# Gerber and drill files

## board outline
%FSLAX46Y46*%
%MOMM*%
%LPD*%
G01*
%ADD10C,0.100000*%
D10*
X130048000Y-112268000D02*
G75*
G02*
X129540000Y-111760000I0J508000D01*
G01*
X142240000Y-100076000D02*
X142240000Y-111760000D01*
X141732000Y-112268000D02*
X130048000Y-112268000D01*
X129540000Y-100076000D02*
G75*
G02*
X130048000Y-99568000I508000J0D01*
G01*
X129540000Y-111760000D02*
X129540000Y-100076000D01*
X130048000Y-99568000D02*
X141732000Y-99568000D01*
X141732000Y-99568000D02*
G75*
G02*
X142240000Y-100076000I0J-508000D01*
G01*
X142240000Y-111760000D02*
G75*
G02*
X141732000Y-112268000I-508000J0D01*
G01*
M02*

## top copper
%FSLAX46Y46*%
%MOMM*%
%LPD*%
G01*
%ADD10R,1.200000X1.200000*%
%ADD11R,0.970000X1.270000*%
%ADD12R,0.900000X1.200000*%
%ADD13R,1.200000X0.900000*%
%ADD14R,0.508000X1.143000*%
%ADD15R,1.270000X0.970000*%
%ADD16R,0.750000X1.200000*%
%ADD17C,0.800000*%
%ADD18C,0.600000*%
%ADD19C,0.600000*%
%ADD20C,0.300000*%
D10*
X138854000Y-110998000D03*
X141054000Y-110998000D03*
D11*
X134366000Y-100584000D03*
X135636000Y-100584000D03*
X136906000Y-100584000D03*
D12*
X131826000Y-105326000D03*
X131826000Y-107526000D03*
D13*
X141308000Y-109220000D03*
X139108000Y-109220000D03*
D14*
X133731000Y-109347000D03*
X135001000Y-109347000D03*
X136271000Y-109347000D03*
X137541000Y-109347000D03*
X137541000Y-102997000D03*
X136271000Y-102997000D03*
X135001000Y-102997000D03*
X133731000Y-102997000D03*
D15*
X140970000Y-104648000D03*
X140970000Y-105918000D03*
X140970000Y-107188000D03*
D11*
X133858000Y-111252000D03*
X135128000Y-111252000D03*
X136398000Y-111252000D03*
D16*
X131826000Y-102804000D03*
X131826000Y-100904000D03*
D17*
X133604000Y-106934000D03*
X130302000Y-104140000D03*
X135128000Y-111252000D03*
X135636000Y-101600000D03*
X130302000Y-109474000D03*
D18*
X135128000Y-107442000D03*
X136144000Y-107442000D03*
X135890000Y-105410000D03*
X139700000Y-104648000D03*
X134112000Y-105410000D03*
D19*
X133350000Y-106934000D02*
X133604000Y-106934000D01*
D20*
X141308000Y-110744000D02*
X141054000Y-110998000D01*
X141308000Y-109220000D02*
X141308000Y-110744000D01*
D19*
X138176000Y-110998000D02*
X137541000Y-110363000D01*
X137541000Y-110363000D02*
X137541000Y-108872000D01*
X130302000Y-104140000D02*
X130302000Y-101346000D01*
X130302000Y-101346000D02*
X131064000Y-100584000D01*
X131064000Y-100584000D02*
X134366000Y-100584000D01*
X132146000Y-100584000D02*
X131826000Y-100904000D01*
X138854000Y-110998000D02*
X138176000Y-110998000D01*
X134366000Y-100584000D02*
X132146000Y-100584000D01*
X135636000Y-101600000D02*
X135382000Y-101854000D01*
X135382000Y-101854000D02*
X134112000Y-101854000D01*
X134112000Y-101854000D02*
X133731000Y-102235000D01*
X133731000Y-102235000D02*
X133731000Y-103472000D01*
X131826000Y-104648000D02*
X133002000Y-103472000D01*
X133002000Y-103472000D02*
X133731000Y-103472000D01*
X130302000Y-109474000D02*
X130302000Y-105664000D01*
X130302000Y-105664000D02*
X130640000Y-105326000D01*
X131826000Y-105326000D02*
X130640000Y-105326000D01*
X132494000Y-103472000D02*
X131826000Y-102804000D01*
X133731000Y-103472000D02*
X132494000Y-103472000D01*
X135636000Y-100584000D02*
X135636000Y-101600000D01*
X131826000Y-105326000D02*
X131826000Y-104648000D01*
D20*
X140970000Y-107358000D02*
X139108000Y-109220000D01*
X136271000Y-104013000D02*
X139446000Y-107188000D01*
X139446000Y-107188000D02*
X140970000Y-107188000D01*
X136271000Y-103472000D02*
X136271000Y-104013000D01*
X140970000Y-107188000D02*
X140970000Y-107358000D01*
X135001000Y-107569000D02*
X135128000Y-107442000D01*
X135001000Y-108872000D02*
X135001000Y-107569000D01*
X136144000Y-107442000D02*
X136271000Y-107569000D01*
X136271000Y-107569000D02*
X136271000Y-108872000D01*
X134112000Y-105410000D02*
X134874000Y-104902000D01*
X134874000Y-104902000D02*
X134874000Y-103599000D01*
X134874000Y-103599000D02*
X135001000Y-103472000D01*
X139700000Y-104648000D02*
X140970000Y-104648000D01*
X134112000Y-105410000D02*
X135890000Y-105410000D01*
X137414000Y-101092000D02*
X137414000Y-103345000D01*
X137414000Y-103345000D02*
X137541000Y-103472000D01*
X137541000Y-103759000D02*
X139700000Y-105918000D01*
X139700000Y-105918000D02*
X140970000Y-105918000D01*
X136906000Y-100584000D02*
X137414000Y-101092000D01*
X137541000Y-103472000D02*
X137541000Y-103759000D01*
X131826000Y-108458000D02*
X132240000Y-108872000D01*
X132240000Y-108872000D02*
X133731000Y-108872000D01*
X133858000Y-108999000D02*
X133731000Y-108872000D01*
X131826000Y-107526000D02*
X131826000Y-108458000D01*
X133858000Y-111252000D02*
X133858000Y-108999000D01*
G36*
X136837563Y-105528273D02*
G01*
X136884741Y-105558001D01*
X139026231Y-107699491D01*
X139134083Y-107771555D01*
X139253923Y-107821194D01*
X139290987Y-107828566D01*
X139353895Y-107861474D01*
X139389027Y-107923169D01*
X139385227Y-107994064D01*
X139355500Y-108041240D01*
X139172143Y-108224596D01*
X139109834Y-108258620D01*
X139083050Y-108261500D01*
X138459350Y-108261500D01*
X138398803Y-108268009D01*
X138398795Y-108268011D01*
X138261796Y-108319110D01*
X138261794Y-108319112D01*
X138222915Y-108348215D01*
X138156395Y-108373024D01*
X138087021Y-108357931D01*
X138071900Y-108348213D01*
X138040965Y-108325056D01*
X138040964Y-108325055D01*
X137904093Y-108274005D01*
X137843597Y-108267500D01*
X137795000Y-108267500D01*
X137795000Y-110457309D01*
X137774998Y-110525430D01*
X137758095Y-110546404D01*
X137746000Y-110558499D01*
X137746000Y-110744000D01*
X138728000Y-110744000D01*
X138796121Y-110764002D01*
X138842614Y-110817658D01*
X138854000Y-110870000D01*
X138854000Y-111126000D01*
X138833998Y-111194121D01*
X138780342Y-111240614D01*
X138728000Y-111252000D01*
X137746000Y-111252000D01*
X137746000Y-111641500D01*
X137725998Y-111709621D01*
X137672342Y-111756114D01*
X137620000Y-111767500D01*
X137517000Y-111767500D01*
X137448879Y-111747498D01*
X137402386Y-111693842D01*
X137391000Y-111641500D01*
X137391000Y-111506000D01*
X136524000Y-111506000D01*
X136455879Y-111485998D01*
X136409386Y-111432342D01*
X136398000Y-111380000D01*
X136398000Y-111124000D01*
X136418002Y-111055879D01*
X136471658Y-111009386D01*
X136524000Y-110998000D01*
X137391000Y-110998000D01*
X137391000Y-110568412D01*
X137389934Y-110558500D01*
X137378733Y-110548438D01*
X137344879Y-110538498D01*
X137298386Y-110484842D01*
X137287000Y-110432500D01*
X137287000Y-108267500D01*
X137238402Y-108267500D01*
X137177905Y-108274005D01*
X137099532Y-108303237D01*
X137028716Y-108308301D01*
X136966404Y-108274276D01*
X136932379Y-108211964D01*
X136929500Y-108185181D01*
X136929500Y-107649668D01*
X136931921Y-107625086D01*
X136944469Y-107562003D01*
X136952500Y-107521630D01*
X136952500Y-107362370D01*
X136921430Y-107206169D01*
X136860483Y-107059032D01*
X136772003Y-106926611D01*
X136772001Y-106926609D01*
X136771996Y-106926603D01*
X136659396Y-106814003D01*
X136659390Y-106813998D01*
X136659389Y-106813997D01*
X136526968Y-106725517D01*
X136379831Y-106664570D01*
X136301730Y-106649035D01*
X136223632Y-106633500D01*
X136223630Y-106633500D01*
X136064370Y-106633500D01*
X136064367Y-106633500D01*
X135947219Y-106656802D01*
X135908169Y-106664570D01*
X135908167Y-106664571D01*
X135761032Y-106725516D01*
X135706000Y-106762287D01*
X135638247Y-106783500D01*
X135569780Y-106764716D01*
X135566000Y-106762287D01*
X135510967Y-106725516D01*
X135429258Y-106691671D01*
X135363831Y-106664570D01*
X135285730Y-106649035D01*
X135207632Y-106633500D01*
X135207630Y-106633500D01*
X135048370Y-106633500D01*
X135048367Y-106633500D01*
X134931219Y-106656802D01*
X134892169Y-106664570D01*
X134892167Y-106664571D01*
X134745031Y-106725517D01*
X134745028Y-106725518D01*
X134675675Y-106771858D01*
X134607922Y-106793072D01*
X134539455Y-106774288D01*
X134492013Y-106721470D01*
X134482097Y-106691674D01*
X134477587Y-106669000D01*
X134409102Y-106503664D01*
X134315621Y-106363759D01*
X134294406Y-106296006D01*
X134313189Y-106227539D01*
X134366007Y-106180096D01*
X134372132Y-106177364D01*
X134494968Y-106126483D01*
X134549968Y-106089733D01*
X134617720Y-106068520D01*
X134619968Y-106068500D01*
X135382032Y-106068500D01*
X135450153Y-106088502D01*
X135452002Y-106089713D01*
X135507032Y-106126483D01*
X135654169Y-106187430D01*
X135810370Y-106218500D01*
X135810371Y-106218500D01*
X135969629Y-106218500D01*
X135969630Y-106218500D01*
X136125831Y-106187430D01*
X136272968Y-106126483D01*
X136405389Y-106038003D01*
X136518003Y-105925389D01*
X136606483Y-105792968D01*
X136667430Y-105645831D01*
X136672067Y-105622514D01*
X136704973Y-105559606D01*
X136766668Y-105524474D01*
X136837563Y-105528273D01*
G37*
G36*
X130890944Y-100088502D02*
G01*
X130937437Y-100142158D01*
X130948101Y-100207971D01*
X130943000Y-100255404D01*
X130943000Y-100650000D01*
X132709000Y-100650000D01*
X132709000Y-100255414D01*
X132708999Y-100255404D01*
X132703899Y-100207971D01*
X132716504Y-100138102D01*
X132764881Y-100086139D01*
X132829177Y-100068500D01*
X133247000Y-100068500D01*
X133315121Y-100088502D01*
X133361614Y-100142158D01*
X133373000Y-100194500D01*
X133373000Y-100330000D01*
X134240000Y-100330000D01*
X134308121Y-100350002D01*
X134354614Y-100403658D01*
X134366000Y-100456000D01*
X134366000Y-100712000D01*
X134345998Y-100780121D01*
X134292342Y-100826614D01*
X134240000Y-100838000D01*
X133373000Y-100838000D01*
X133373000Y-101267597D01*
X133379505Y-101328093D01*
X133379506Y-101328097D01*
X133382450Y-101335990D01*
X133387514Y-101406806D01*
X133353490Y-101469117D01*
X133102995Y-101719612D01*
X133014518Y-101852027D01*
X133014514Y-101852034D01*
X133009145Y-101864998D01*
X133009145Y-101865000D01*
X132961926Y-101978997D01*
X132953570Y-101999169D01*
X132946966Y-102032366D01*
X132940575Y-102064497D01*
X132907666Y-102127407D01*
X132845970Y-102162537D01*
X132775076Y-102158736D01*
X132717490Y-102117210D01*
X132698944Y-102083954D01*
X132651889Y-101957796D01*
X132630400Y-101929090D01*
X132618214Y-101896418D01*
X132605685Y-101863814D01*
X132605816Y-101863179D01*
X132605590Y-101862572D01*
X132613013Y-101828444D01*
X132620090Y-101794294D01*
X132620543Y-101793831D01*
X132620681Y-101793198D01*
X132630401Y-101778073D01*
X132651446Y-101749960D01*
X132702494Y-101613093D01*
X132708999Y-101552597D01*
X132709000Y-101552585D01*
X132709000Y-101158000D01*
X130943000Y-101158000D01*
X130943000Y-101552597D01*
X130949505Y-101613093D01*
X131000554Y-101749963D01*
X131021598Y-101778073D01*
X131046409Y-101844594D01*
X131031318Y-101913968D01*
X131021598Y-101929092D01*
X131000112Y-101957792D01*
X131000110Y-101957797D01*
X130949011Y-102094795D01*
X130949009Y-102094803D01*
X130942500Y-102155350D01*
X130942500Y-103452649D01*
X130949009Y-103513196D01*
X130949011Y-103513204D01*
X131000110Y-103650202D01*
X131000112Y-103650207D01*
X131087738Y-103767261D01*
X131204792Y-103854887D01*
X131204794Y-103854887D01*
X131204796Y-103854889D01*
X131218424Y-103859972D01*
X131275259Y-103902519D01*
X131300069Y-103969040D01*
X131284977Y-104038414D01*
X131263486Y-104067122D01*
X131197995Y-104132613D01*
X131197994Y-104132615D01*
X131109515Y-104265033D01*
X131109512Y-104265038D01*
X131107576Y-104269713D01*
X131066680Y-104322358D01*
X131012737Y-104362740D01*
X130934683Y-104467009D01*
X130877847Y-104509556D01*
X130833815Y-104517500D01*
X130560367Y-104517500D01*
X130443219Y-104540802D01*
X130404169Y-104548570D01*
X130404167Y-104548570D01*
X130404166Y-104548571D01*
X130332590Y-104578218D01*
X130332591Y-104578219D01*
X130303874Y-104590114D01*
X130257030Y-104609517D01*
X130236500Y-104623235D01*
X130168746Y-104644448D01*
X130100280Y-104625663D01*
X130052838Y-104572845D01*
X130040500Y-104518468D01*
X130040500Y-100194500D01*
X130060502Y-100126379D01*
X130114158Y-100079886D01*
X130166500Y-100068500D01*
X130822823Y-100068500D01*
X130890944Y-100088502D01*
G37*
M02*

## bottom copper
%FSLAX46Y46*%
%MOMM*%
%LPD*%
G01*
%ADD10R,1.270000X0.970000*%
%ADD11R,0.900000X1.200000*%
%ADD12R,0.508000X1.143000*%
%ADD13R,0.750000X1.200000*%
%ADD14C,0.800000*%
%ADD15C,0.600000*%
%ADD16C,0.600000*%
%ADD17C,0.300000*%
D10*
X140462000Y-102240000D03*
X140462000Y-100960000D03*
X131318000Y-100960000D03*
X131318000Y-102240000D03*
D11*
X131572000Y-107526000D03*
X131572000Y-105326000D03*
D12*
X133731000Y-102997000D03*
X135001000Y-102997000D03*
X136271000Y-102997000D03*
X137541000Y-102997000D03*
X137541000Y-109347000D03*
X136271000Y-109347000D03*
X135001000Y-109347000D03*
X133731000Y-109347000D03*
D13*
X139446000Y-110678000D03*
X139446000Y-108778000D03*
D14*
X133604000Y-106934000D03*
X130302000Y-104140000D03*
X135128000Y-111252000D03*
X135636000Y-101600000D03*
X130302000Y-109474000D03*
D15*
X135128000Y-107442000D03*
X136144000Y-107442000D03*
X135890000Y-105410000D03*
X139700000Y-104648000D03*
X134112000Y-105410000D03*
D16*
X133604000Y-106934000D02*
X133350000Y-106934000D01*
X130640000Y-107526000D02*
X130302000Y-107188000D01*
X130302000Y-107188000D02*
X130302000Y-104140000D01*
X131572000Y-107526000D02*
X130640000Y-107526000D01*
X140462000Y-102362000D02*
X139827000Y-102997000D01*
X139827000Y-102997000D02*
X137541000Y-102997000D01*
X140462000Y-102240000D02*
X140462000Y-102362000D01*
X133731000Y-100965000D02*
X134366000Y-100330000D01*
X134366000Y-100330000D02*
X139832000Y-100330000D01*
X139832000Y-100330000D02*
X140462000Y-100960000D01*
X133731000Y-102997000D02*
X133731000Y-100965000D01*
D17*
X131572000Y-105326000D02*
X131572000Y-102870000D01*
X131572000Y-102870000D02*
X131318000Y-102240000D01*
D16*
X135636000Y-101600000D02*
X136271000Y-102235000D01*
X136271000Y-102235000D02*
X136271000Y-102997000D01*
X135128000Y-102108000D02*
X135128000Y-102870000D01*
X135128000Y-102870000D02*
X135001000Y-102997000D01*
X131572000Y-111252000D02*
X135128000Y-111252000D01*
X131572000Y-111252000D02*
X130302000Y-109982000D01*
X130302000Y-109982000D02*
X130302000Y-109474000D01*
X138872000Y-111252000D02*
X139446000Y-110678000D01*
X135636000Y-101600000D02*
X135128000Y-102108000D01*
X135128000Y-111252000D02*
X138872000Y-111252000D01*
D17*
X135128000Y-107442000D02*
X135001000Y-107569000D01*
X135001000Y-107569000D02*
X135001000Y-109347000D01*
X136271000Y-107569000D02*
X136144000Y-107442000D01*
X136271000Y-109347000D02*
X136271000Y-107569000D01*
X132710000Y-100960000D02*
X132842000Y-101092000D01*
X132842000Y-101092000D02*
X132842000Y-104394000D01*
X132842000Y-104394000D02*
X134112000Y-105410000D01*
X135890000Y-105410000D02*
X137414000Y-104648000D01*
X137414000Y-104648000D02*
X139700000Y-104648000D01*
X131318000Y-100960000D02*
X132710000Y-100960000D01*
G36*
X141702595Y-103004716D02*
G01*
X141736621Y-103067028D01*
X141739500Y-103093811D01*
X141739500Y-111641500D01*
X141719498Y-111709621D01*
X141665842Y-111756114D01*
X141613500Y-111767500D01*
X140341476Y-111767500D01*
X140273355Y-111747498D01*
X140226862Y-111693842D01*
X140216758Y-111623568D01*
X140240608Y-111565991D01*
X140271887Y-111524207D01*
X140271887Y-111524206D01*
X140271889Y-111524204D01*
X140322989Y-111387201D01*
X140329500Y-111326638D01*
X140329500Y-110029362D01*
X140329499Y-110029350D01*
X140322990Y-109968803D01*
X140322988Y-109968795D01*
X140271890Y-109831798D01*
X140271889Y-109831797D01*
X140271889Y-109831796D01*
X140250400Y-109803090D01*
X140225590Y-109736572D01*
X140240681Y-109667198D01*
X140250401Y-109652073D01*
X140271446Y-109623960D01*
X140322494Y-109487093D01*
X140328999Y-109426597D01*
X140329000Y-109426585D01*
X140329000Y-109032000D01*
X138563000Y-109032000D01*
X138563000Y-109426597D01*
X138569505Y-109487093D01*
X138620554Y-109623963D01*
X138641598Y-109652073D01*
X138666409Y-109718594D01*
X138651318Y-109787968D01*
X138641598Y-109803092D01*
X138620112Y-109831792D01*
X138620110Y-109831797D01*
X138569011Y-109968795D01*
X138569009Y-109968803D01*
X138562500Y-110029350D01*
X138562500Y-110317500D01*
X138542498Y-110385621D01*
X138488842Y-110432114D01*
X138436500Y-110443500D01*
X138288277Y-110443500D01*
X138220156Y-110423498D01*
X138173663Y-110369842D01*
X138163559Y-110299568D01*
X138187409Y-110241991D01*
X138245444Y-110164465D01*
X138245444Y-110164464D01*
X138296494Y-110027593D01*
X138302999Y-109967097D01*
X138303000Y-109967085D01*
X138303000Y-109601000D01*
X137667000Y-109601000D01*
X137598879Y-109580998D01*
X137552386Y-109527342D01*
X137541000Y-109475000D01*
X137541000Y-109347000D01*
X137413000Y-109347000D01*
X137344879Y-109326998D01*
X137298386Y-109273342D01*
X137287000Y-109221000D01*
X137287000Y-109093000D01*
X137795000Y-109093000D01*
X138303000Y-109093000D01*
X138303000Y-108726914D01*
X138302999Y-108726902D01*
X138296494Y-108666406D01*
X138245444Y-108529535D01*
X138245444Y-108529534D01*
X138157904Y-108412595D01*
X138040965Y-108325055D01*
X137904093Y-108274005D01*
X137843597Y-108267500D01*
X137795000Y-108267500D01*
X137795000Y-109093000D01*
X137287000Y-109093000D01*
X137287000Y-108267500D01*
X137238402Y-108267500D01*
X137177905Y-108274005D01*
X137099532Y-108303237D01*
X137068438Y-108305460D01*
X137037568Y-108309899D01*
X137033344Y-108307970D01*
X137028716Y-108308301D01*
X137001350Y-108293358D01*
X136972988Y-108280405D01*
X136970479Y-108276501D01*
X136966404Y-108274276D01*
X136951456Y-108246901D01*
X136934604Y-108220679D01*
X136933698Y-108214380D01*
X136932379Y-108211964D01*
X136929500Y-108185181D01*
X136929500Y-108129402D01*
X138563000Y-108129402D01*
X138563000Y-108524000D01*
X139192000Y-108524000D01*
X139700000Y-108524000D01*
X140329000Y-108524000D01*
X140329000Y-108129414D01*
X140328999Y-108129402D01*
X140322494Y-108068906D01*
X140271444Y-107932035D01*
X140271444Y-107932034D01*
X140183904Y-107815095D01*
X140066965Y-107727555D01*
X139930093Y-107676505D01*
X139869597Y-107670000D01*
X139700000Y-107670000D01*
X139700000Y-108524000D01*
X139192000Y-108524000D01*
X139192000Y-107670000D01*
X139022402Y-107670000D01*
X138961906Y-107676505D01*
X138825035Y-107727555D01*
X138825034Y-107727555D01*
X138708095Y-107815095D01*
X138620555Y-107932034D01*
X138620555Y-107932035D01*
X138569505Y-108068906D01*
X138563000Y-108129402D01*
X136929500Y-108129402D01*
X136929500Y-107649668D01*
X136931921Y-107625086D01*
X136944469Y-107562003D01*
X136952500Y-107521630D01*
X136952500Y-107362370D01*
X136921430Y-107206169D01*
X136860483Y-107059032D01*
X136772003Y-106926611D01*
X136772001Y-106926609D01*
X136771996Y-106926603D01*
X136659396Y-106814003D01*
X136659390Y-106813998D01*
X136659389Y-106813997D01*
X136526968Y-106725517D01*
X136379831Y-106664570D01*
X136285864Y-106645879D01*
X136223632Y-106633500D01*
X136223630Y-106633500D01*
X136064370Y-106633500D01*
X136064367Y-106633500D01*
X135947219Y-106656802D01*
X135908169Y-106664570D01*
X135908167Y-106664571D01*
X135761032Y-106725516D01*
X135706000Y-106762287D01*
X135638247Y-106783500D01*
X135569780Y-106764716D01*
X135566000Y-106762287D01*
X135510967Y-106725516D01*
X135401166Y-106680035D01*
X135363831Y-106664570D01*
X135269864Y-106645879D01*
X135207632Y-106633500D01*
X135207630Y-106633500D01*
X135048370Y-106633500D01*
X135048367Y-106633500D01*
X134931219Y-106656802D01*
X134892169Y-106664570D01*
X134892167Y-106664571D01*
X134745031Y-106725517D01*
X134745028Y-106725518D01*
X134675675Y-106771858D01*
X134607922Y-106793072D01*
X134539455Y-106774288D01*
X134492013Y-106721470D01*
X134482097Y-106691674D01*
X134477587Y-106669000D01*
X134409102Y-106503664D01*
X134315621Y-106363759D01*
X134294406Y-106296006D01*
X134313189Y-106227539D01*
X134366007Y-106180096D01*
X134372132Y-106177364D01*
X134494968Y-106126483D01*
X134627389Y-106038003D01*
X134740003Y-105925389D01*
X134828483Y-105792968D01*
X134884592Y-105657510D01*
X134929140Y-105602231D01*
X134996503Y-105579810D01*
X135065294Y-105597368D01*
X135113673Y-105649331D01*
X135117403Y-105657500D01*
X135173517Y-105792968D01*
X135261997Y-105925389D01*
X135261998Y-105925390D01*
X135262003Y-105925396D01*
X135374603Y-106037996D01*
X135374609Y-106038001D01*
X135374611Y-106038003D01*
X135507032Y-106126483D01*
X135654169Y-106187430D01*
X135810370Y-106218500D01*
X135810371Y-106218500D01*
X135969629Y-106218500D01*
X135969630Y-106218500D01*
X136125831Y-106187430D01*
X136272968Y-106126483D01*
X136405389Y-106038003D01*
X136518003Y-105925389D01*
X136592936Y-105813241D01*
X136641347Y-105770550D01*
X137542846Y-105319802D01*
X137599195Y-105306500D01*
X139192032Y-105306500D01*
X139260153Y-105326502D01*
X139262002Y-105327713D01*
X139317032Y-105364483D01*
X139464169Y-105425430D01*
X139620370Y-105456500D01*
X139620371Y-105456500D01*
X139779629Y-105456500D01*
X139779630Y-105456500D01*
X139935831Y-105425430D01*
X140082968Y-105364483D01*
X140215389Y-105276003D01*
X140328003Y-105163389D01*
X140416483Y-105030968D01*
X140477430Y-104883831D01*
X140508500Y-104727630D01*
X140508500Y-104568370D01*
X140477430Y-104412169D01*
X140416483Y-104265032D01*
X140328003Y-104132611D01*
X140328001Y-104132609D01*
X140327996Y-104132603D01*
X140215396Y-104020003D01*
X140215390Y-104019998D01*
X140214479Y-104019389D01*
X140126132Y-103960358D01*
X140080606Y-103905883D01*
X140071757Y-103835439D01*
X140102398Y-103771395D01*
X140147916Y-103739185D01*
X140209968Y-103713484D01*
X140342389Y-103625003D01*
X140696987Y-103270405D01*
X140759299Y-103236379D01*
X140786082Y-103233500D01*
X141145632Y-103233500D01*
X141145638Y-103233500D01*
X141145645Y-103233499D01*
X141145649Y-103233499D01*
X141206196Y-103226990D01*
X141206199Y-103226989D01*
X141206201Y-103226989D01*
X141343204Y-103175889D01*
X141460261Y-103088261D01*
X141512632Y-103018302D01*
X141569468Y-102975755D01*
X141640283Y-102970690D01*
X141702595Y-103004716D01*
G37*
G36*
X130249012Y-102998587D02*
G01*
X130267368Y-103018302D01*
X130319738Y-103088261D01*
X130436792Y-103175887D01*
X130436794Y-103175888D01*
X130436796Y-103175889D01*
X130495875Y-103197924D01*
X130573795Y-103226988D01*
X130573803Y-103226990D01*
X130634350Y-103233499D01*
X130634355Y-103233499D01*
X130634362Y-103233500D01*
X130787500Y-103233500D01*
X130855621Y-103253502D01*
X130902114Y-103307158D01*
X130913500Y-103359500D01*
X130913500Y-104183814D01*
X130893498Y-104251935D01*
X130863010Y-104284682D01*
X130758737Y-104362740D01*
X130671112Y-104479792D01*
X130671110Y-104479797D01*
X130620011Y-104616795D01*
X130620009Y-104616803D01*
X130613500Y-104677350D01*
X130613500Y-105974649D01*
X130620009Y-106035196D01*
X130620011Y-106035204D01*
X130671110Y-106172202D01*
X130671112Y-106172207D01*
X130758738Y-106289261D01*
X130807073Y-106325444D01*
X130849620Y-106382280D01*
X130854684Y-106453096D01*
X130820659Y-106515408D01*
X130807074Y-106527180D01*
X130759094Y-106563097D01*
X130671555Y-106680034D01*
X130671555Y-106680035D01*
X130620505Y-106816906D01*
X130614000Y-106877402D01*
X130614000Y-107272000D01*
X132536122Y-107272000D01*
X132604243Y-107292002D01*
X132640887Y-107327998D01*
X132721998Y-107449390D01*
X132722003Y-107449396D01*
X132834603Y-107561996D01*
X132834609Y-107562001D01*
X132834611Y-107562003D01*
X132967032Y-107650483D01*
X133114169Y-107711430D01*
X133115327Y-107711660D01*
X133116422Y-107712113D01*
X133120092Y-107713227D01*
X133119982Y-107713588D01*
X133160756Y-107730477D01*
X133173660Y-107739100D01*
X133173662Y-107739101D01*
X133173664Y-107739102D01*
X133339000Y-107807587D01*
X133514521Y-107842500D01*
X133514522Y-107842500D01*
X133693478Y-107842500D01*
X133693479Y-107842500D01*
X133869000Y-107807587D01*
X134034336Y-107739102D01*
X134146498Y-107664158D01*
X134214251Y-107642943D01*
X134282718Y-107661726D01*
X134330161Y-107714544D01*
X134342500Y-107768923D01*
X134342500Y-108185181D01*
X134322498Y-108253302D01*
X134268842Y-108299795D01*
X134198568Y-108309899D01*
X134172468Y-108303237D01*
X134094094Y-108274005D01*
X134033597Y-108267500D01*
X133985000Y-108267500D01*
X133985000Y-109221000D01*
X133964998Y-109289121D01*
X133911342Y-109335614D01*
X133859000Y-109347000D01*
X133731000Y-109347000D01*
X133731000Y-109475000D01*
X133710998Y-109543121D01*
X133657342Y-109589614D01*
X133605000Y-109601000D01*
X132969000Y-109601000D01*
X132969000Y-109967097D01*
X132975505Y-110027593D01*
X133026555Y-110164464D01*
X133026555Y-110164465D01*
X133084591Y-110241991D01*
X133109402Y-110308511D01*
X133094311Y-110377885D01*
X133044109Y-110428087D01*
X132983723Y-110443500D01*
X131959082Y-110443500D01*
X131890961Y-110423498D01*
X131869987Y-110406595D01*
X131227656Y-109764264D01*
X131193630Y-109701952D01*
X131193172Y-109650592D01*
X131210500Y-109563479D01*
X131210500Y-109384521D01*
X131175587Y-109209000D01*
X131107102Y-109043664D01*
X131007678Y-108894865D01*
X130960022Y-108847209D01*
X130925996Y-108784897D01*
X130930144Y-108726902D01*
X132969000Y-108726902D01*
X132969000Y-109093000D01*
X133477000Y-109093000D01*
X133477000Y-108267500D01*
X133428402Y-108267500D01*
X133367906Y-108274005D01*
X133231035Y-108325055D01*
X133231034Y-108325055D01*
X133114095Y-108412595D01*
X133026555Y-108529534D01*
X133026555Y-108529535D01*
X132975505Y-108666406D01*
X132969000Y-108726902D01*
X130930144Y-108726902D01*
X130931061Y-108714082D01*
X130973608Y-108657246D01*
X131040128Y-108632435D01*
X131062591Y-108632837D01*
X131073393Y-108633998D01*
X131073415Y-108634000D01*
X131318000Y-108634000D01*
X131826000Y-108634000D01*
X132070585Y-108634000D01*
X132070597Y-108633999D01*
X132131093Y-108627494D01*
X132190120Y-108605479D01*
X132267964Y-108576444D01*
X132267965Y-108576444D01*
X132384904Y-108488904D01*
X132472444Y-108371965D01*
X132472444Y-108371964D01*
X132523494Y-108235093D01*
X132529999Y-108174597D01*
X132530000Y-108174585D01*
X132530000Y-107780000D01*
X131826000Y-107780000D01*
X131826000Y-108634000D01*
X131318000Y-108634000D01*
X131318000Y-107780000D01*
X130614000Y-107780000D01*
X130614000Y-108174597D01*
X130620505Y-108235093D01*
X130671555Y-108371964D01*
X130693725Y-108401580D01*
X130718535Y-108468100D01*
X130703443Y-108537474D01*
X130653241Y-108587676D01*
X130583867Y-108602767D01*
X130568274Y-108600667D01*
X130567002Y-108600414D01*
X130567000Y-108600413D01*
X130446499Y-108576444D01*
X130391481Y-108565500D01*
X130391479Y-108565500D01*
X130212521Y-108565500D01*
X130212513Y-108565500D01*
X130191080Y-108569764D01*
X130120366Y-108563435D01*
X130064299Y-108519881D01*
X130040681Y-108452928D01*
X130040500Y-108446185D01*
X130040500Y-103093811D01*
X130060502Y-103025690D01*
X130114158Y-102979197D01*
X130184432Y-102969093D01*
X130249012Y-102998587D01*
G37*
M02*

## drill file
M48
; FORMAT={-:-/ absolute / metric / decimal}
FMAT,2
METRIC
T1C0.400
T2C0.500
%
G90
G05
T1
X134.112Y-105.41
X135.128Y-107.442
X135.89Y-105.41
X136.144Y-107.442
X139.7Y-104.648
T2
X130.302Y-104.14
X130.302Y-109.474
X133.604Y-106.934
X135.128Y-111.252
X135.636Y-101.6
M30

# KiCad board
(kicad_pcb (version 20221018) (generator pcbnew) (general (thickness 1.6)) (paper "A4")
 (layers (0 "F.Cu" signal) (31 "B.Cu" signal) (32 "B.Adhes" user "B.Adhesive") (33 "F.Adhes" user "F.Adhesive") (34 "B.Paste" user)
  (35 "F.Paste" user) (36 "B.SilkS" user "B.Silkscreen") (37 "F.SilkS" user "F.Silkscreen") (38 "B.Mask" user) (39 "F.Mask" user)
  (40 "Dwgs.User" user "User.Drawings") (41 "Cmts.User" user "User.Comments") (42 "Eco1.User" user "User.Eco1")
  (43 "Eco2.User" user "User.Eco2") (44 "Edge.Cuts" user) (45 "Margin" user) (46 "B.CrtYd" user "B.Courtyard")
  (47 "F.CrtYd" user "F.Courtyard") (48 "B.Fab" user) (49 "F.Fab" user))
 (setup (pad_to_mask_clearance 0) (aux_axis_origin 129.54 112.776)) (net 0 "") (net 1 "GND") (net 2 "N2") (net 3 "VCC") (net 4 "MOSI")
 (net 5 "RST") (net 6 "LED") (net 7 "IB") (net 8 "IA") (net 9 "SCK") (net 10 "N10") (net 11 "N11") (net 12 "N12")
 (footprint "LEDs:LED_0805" (layer "F.Cu") (at 139.954 110.998)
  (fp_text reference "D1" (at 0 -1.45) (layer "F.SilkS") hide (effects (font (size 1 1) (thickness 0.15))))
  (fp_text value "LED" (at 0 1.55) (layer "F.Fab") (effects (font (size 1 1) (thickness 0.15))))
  (pad "1" smd rect (at -1.1 0 180) (size 1.2 1.2) (layers "F.Cu" "F.Paste" "F.Mask") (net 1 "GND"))
  (pad "2" smd rect (at 1.1 0 180) (size 1.2 1.2) (layers "F.Cu" "F.Paste" "F.Mask") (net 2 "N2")))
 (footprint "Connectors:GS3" (layer "F.Cu") (at 135.636 100.584 90)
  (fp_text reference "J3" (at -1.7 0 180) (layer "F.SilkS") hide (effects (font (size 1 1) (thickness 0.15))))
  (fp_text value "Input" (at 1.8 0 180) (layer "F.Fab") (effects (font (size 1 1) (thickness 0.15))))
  (pad "1" smd rect (at 0 -1.27 90) (size 1.27 0.97) (layers "F.Cu" "F.Paste" "F.Mask") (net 1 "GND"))
  (pad "2" smd rect (at 0 0 90) (size 1.27 0.97) (layers "F.Cu" "F.Paste" "F.Mask") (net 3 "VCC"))
  (pad "3" smd rect (at 0 1.27 90) (size 1.27 0.97) (layers "F.Cu" "F.Paste" "F.Mask") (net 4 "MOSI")))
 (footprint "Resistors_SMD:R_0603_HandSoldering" (layer "F.Cu") (at 131.826 106.426 -90)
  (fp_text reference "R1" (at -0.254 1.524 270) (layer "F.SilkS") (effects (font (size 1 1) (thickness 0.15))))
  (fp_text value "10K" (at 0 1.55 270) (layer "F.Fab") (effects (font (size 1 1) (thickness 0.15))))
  (pad "1" smd rect (at -1.1 0 270) (size 1.2 0.9) (layers "F.Cu" "F.Paste" "F.Mask") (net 3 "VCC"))
  (pad "2" smd rect (at 1.1 0 270) (size 1.2 0.9) (layers "F.Cu" "F.Paste" "F.Mask") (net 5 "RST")))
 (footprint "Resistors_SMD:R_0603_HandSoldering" (layer "F.Cu") (at 140.208 109.22 180)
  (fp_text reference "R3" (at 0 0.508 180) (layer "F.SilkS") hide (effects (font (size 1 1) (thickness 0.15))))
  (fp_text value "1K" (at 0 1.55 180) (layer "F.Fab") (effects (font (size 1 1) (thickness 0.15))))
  (pad "1" smd rect (at -1.1 0 180) (size 1.2 0.9) (layers "F.Cu" "F.Paste" "F.Mask") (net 2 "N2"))
  (pad "2" smd rect (at 1.1 0 180) (size 1.2 0.9) (layers "F.Cu" "F.Paste" "F.Mask") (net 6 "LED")))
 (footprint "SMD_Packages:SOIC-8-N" (layer "F.Cu") (at 135.636 106.172)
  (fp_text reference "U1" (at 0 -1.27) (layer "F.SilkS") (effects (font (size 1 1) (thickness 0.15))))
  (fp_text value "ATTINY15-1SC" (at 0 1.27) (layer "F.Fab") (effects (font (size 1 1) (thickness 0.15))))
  (pad "1" smd rect (at -1.905 3.175) (size 0.508 1.143) (layers "F.Cu" "F.Paste" "F.Mask") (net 5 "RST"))
  (pad "2" smd rect (at -0.635 3.175) (size 0.508 1.143) (layers "F.Cu" "F.Paste" "F.Mask") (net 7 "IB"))
  (pad "3" smd rect (at 0.635 3.175) (size 0.508 1.143) (layers "F.Cu" "F.Paste" "F.Mask") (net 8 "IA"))
  (pad "4" smd rect (at 1.905 3.175) (size 0.508 1.143) (layers "F.Cu" "F.Paste" "F.Mask") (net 1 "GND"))
  (pad "5" smd rect (at 1.905 -3.175) (size 0.508 1.143) (layers "F.Cu" "F.Paste" "F.Mask") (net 4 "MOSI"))
  (pad "6" smd rect (at 0.635 -3.175) (size 0.508 1.143) (layers "F.Cu" "F.Paste" "F.Mask") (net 6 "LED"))
  (pad "7" smd rect (at -0.635 -3.175) (size 0.508 1.143) (layers "F.Cu" "F.Paste" "F.Mask") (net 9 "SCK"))
  (pad "8" smd rect (at -1.905 -3.175) (size 0.508 1.143) (layers "F.Cu" "F.Paste" "F.Mask") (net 3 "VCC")))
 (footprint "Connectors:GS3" (layer "F.Cu") (at 140.97 105.918)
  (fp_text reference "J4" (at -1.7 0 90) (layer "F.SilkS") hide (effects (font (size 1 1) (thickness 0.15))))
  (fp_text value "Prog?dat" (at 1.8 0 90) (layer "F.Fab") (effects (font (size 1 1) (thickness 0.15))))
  (pad "1" smd rect (at 0 -1.27) (size 1.27 0.97) (layers "F.Cu" "F.Paste" "F.Mask") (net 9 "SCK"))
  (pad "2" smd rect (at 0 0) (size 1.27 0.97) (layers "F.Cu" "F.Paste" "F.Mask") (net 4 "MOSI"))
  (pad "3" smd rect (at 0 1.27) (size 1.27 0.97) (layers "F.Cu" "F.Paste" "F.Mask") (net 6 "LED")))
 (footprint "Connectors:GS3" (layer "F.Cu") (at 135.128 111.252 90)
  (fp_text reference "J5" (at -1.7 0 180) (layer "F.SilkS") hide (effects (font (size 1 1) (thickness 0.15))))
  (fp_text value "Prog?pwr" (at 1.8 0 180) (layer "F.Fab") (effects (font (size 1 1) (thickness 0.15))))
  (pad "1" smd rect (at 0 -1.27 90) (size 1.27 0.97) (layers "F.Cu" "F.Paste" "F.Mask") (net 5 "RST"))
  (pad "2" smd rect (at 0 0 90) (size 1.27 0.97) (layers "F.Cu" "F.Paste" "F.Mask") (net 3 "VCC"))
  (pad "3" smd rect (at 0 1.27 90) (size 1.27 0.97) (layers "F.Cu" "F.Paste" "F.Mask") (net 1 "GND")))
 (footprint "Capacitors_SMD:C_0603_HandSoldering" (layer "F.Cu") (at 131.826 101.854 90)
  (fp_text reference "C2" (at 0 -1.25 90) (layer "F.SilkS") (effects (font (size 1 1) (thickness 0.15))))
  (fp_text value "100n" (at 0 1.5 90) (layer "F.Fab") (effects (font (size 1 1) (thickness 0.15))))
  (pad "1" smd rect (at -0.95 0 90) (size 1.2 0.75) (layers "F.Cu" "F.Paste" "F.Mask") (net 3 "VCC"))
  (pad "2" smd rect (at 0.95 0 90) (size 1.2 0.75) (layers "F.Cu" "F.Paste" "F.Mask") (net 1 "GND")))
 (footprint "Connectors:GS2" (layer "B.Cu") (at 140.462 101.6)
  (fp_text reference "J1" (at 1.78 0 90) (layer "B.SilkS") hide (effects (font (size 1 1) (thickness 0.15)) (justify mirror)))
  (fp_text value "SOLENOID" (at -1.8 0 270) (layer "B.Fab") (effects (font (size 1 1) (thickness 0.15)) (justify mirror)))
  (pad "1" smd rect (at 0 0.64) (size 1.27 0.97) (layers "B.Cu" "B.Paste" "B.Mask") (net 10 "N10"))
  (pad "2" smd rect (at 0 -0.64) (size 1.27 0.97) (layers "B.Cu" "B.Paste" "B.Mask") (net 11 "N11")))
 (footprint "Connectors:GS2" (layer "B.Cu") (at 131.318 101.6 180)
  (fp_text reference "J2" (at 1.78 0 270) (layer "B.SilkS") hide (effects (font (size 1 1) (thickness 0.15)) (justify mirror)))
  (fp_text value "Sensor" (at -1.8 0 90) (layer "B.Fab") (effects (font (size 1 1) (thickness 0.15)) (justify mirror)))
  (pad "1" smd rect (at 0 0.64 180) (size 1.27 0.97) (layers "B.Cu" "B.Paste" "B.Mask") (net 9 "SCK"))
  (pad "2" smd rect (at 0 -0.64 180) (size 1.27 0.97) (layers "B.Cu" "B.Paste" "B.Mask") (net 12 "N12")))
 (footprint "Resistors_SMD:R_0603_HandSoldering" (layer "B.Cu") (at 131.572 106.426 90)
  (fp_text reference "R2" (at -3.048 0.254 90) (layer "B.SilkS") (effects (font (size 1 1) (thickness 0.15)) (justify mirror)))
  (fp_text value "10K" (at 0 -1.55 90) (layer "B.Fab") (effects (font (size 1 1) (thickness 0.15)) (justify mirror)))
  (pad "1" smd rect (at -1.1 0 90) (size 1.2 0.9) (layers "B.Cu" "B.Paste" "B.Mask") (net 1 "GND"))
  (pad "2" smd rect (at 1.1 0 90) (size 1.2 0.9) (layers "B.Cu" "B.Paste" "B.Mask") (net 12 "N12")))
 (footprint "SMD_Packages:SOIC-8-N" (layer "B.Cu") (at 135.636 106.172)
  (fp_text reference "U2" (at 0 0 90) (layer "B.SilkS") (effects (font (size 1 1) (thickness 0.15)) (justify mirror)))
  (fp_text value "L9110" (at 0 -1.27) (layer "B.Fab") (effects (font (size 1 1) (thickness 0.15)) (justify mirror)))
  (pad "1" smd rect (at -1.905 -3.175) (size 0.508 1.143) (layers "B.Cu" "B.Paste" "B.Mask") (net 11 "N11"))
  (pad "2" smd rect (at -0.635 -3.175) (size 0.508 1.143) (layers "B.Cu" "B.Paste" "B.Mask") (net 3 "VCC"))
  (pad "3" smd rect (at 0.635 -3.175) (size 0.508 1.143) (layers "B.Cu" "B.Paste" "B.Mask") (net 3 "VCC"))
  (pad "4" smd rect (at 1.905 -3.175) (size 0.508 1.143) (layers "B.Cu" "B.Paste" "B.Mask") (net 10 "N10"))
  (pad "5" smd rect (at 1.905 3.175) (size 0.508 1.143) (layers "B.Cu" "B.Paste" "B.Mask") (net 1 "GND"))
  (pad "6" smd rect (at 0.635 3.175) (size 0.508 1.143) (layers "B.Cu" "B.Paste" "B.Mask") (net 8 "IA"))
  (pad "7" smd rect (at -0.635 3.175) (size 0.508 1.143) (layers "B.Cu" "B.Paste" "B.Mask") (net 7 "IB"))
  (pad "8" smd rect (at -1.905 3.175) (size 0.508 1.143) (layers "B.Cu" "B.Paste" "B.Mask") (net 1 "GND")))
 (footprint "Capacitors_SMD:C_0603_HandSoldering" (layer "B.Cu") (at 139.446 109.728 90)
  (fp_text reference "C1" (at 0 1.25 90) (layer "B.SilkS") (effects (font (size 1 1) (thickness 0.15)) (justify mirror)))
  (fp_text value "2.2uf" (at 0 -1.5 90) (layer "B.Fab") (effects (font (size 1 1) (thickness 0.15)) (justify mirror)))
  (pad "1" smd rect (at -0.95 0 90) (size 1.2 0.75) (layers "B.Cu" "B.Paste" "B.Mask") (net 3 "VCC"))
  (pad "2" smd rect (at 0.95 0 90) (size 1.2 0.75) (layers "B.Cu" "B.Paste" "B.Mask") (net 1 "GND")))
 (gr_arc (start 130.048 112.268) (mid 129.68879 112.11921) (end 129.54 111.76) (stroke (width 0.1) (type solid)) (layer "Edge.Cuts"))
 (gr_line (start 142.24 100.076) (end 142.24 111.76) (stroke (width 0.1) (type solid)) (layer "Edge.Cuts"))
 (gr_line (start 141.732 112.268) (end 130.048 112.268) (stroke (width 0.1) (type solid)) (layer "Edge.Cuts"))
 (gr_arc (start 129.54 100.076) (mid 129.68879 99.71679) (end 130.048 99.568) (stroke (width 0.1) (type solid)) (layer "Edge.Cuts"))
 (gr_line (start 129.54 111.76) (end 129.54 100.076) (stroke (width 0.1) (type solid)) (layer "Edge.Cuts"))
 (gr_line (start 130.048 99.568) (end 141.732 99.568) (stroke (width 0.1) (type solid)) (layer "Edge.Cuts"))
 (gr_arc (start 141.732 99.568) (mid 142.09121 99.71679) (end 142.24 100.076) (stroke (width 0.1) (type solid)) (layer "Edge.Cuts"))
 (gr_arc (start 142.24 111.76) (mid 142.09121 112.11921) (end 141.732 112.268) (stroke (width 0.1) (type solid)) (layer "Edge.Cuts"))
 (segment (start 133.35 106.934) (end 133.604 106.934) (width 0.6) (layer "F.Cu") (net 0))
 (via (at 133.604 106.934) (size 0.8) (drill 0.5) (layers "F.Cu" "B.Cu") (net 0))
 (segment (start 133.604 106.934) (end 133.35 106.934) (width 0.6) (layer "B.Cu") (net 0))
 (segment (start 141.308 110.744) (end 141.054 110.998) (width 0.3) (layer "F.Cu") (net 2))
 (segment (start 141.308 109.22) (end 141.308 110.744) (width 0.3) (layer "F.Cu") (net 2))
 (segment (start 138.176 110.998) (end 137.541 110.363) (width 0.6) (layer "F.Cu") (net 1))
 (segment (start 137.541 110.363) (end 137.541 108.872) (width 0.6) (layer "F.Cu") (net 1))
 (segment (start 130.302 104.14) (end 130.302 101.346) (width 0.6) (layer "F.Cu") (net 1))
 (segment (start 130.302 101.346) (end 131.064 100.584) (width 0.6) (layer "F.Cu") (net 1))
 (segment (start 131.064 100.584) (end 134.366 100.584) (width 0.6) (layer "F.Cu") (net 1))
 (segment (start 132.146 100.584) (end 131.826 100.904) (width 0.6) (layer "F.Cu") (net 1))
 (segment (start 138.854 110.998) (end 138.176 110.998) (width 0.6) (layer "F.Cu") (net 1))
 (segment (start 134.366 100.584) (end 132.146 100.584) (width 0.6) (layer "F.Cu") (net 1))
 (via (at 130.302 104.14) (size 0.8) (drill 0.5) (layers "F.Cu" "B.Cu") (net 1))
 (segment (start 130.64 107.526) (end 130.302 107.188) (width 0.6) (layer "B.Cu") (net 1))
 (segment (start 130.302 107.188) (end 130.302 104.14) (width 0.6) (layer "B.Cu") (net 1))
 (segment (start 131.572 107.526) (end 130.64 107.526) (width 0.6) (layer "B.Cu") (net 1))
 (segment (start 140.462 102.362) (end 139.827 102.997) (width 0.6) (layer "B.Cu") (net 10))
 (segment (start 139.827 102.997) (end 137.541 102.997) (width 0.6) (layer "B.Cu") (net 10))
 (segment (start 140.462 102.24) (end 140.462 102.362) (width 0.6) (layer "B.Cu") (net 10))
 (segment (start 133.731 100.965) (end 134.366 100.33) (width 0.6) (layer "B.Cu") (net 11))
 (segment (start 134.366 100.33) (end 139.832 100.33) (width 0.6) (layer "B.Cu") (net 11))
 (segment (start 139.832 100.33) (end 140.462 100.96) (width 0.6) (layer "B.Cu") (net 11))
 (segment (start 133.731 102.997) (end 133.731 100.965) (width 0.6) (layer "B.Cu") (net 11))
 (segment (start 131.572 105.326) (end 131.572 102.87) (width 0.3) (layer "B.Cu") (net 12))
 (segment (start 131.572 102.87) (end 131.318 102.24) (width 0.3) (layer "B.Cu") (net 12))
 (segment (start 135.636 101.6) (end 135.382 101.854) (width 0.6) (layer "F.Cu") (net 3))
 (segment (start 135.382 101.854) (end 134.112 101.854) (width 0.6) (layer "F.Cu") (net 3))
 (segment (start 134.112 101.854) (end 133.731 102.235) (width 0.6) (layer "F.Cu") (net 3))
 (segment (start 133.731 102.235) (end 133.731 103.472) (width 0.6) (layer "F.Cu") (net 3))
 (segment (start 131.826 104.648) (end 133.002 103.472) (width 0.6) (layer "F.Cu") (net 3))
 (segment (start 133.002 103.472) (end 133.731 103.472) (width 0.6) (layer "F.Cu") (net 3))
 (segment (start 130.302 109.474) (end 130.302 105.664) (width 0.6) (layer "F.Cu") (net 3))
 (segment (start 130.302 105.664) (end 130.64 105.326) (width 0.6) (layer "F.Cu") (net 3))
 (segment (start 131.826 105.326) (end 130.64 105.326) (width 0.6) (layer "F.Cu") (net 3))
 (segment (start 132.494 103.472) (end 131.826 102.804) (width 0.6) (layer "F.Cu") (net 3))
 (segment (start 133.731 103.472) (end 132.494 103.472) (width 0.6) (layer "F.Cu") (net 3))
 (segment (start 135.636 100.584) (end 135.636 101.6) (width 0.6) (layer "F.Cu") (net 3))
 (segment (start 131.826 105.326) (end 131.826 104.648) (width 0.6) (layer "F.Cu") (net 3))
 (via (at 135.128 111.252) (size 0.8) (drill 0.5) (layers "F.Cu" "B.Cu") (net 3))
 (via (at 135.636 101.6) (size 0.8) (drill 0.5) (layers "F.Cu" "B.Cu") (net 3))
 (via (at 130.302 109.474) (size 0.8) (drill 0.5) (layers "F.Cu" "B.Cu") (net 3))
 (segment (start 135.636 101.6) (end 136.271 102.235) (width 0.6) (layer "B.Cu") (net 3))
 (segment (start 136.271 102.235) (end 136.271 102.997) (width 0.6) (layer "B.Cu") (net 3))
 (segment (start 135.128 102.108) (end 135.128 102.87) (width 0.6) (layer "B.Cu") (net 3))
 (segment (start 135.128 102.87) (end 135.001 102.997) (width 0.6) (layer "B.Cu") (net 3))
 (segment (start 131.572 111.252) (end 135.128 111.252) (width 0.6) (layer "B.Cu") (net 3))
 (segment (start 131.572 111.252) (end 130.302 109.982) (width 0.6) (layer "B.Cu") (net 3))
 (segment (start 130.302 109.982) (end 130.302 109.474) (width 0.6) (layer "B.Cu") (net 3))
 (segment (start 138.872 111.252) (end 139.446 110.678) (width 0.6) (layer "B.Cu") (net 3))
 (segment (start 135.636 101.6) (end 135.128 102.108) (width 0.6) (layer "B.Cu") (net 3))
 (segment (start 135.128 111.252) (end 138.872 111.252) (width 0.6) (layer "B.Cu") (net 3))
 (segment (start 140.97 107.358) (end 139.108 109.22) (width 0.3) (layer "F.Cu") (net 6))
 (segment (start 136.271 104.013) (end 139.446 107.188) (width 0.3) (layer "F.Cu") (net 6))
 (segment (start 139.446 107.188) (end 140.97 107.188) (width 0.3) (layer "F.Cu") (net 6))
 (segment (start 136.271 103.472) (end 136.271 104.013) (width 0.3) (layer "F.Cu") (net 6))
 (segment (start 140.97 107.188) (end 140.97 107.358) (width 0.3) (layer "F.Cu") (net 6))
 (segment (start 135.001 107.569) (end 135.128 107.442) (width 0.3) (layer "F.Cu") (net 7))
 (segment (start 135.001 108.872) (end 135.001 107.569) (width 0.3) (layer "F.Cu") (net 7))
 (via (at 135.128 107.442) (size 0.6) (drill 0.4) (layers "F.Cu" "B.Cu") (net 7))
 (segment (start 135.128 107.442) (end 135.001 107.569) (width 0.3) (layer "B.Cu") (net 7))
 (segment (start 135.001 107.569) (end 135.001 109.347) (width 0.3) (layer "B.Cu") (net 7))
 (segment (start 136.144 107.442) (end 136.271 107.569) (width 0.3) (layer "F.Cu") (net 8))
 (segment (start 136.271 107.569) (end 136.271 108.872) (width 0.3) (layer "F.Cu") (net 8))
 (via (at 136.144 107.442) (size 0.6) (drill 0.4) (layers "F.Cu" "B.Cu") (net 8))
 (segment (start 136.271 107.569) (end 136.144 107.442) (width 0.3) (layer "B.Cu") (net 8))
 (segment (start 136.271 109.347) (end 136.271 107.569) (width 0.3) (layer "B.Cu") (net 8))
 (segment (start 134.112 105.41) (end 134.874 104.902) (width 0.3) (layer "F.Cu") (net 9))
 (segment (start 134.874 104.902) (end 134.874 103.599) (width 0.3) (layer "F.Cu") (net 9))
 (segment (start 134.874 103.599) (end 135.001 103.472) (width 0.3) (layer "F.Cu") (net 9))
 (segment (start 139.7 104.648) (end 140.97 104.648) (width 0.3) (layer "F.Cu") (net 9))
 (segment (start 134.112 105.41) (end 135.89 105.41) (width 0.3) (layer "F.Cu") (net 9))
 (via (at 135.89 105.41) (size 0.6) (drill 0.4) (layers "F.Cu" "B.Cu") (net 9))
 (via (at 139.7 104.648) (size 0.6) (drill 0.4) (layers "F.Cu" "B.Cu") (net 9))
 (via (at 134.112 105.41) (size 0.6) (drill 0.4) (layers "F.Cu" "B.Cu") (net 9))
 (segment (start 132.71 100.96) (end 132.842 101.092) (width 0.3) (layer "B.Cu") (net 9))
 (segment (start 132.842 101.092) (end 132.842 104.394) (width 0.3) (layer "B.Cu") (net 9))
 (segment (start 132.842 104.394) (end 134.112 105.41) (width 0.3) (layer "B.Cu") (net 9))
 (segment (start 135.89 105.41) (end 137.414 104.648) (width 0.3) (layer "B.Cu") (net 9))
 (segment (start 137.414 104.648) (end 139.7 104.648) (width 0.3) (layer "B.Cu") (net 9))
 (segment (start 131.318 100.96) (end 132.71 100.96) (width 0.3) (layer "B.Cu") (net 9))
 (segment (start 137.414 101.092) (end 137.414 103.345) (width 0.3) (layer "F.Cu") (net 4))
 (segment (start 137.414 103.345) (end 137.541 103.472) (width 0.3) (layer "F.Cu") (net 4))
 (segment (start 137.541 103.759) (end 139.7 105.918) (width 0.3) (layer "F.Cu") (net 4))
 (segment (start 139.7 105.918) (end 140.97 105.918) (width 0.3) (layer "F.Cu") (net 4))
 (segment (start 136.906 100.584) (end 137.414 101.092) (width 0.3) (layer "F.Cu") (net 4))
 (segment (start 137.541 103.472) (end 137.541 103.759) (width 0.3) (layer "F.Cu") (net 4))
 (segment (start 131.826 108.458) (end 132.24 108.872) (width 0.3) (layer "F.Cu") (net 5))
 (segment (start 132.24 108.872) (end 133.731 108.872) (width 0.3) (layer "F.Cu") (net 5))
 (segment (start 133.858 108.999) (end 133.731 108.872) (width 0.3) (layer "F.Cu") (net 5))
 (segment (start 131.826 107.526) (end 131.826 108.458) (width 0.3) (layer "F.Cu") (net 5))
 (segment (start 133.858 111.252) (end 133.858 108.999) (width 0.3) (layer "F.Cu") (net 5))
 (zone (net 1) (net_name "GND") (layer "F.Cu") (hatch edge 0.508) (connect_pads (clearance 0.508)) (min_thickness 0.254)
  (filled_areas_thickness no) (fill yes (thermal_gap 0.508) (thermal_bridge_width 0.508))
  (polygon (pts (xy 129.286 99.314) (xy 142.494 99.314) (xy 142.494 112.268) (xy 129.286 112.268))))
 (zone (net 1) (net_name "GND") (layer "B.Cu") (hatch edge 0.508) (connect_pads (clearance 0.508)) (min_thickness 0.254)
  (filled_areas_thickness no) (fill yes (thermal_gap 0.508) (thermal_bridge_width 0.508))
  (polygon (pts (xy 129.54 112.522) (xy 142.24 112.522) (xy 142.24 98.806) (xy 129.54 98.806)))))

